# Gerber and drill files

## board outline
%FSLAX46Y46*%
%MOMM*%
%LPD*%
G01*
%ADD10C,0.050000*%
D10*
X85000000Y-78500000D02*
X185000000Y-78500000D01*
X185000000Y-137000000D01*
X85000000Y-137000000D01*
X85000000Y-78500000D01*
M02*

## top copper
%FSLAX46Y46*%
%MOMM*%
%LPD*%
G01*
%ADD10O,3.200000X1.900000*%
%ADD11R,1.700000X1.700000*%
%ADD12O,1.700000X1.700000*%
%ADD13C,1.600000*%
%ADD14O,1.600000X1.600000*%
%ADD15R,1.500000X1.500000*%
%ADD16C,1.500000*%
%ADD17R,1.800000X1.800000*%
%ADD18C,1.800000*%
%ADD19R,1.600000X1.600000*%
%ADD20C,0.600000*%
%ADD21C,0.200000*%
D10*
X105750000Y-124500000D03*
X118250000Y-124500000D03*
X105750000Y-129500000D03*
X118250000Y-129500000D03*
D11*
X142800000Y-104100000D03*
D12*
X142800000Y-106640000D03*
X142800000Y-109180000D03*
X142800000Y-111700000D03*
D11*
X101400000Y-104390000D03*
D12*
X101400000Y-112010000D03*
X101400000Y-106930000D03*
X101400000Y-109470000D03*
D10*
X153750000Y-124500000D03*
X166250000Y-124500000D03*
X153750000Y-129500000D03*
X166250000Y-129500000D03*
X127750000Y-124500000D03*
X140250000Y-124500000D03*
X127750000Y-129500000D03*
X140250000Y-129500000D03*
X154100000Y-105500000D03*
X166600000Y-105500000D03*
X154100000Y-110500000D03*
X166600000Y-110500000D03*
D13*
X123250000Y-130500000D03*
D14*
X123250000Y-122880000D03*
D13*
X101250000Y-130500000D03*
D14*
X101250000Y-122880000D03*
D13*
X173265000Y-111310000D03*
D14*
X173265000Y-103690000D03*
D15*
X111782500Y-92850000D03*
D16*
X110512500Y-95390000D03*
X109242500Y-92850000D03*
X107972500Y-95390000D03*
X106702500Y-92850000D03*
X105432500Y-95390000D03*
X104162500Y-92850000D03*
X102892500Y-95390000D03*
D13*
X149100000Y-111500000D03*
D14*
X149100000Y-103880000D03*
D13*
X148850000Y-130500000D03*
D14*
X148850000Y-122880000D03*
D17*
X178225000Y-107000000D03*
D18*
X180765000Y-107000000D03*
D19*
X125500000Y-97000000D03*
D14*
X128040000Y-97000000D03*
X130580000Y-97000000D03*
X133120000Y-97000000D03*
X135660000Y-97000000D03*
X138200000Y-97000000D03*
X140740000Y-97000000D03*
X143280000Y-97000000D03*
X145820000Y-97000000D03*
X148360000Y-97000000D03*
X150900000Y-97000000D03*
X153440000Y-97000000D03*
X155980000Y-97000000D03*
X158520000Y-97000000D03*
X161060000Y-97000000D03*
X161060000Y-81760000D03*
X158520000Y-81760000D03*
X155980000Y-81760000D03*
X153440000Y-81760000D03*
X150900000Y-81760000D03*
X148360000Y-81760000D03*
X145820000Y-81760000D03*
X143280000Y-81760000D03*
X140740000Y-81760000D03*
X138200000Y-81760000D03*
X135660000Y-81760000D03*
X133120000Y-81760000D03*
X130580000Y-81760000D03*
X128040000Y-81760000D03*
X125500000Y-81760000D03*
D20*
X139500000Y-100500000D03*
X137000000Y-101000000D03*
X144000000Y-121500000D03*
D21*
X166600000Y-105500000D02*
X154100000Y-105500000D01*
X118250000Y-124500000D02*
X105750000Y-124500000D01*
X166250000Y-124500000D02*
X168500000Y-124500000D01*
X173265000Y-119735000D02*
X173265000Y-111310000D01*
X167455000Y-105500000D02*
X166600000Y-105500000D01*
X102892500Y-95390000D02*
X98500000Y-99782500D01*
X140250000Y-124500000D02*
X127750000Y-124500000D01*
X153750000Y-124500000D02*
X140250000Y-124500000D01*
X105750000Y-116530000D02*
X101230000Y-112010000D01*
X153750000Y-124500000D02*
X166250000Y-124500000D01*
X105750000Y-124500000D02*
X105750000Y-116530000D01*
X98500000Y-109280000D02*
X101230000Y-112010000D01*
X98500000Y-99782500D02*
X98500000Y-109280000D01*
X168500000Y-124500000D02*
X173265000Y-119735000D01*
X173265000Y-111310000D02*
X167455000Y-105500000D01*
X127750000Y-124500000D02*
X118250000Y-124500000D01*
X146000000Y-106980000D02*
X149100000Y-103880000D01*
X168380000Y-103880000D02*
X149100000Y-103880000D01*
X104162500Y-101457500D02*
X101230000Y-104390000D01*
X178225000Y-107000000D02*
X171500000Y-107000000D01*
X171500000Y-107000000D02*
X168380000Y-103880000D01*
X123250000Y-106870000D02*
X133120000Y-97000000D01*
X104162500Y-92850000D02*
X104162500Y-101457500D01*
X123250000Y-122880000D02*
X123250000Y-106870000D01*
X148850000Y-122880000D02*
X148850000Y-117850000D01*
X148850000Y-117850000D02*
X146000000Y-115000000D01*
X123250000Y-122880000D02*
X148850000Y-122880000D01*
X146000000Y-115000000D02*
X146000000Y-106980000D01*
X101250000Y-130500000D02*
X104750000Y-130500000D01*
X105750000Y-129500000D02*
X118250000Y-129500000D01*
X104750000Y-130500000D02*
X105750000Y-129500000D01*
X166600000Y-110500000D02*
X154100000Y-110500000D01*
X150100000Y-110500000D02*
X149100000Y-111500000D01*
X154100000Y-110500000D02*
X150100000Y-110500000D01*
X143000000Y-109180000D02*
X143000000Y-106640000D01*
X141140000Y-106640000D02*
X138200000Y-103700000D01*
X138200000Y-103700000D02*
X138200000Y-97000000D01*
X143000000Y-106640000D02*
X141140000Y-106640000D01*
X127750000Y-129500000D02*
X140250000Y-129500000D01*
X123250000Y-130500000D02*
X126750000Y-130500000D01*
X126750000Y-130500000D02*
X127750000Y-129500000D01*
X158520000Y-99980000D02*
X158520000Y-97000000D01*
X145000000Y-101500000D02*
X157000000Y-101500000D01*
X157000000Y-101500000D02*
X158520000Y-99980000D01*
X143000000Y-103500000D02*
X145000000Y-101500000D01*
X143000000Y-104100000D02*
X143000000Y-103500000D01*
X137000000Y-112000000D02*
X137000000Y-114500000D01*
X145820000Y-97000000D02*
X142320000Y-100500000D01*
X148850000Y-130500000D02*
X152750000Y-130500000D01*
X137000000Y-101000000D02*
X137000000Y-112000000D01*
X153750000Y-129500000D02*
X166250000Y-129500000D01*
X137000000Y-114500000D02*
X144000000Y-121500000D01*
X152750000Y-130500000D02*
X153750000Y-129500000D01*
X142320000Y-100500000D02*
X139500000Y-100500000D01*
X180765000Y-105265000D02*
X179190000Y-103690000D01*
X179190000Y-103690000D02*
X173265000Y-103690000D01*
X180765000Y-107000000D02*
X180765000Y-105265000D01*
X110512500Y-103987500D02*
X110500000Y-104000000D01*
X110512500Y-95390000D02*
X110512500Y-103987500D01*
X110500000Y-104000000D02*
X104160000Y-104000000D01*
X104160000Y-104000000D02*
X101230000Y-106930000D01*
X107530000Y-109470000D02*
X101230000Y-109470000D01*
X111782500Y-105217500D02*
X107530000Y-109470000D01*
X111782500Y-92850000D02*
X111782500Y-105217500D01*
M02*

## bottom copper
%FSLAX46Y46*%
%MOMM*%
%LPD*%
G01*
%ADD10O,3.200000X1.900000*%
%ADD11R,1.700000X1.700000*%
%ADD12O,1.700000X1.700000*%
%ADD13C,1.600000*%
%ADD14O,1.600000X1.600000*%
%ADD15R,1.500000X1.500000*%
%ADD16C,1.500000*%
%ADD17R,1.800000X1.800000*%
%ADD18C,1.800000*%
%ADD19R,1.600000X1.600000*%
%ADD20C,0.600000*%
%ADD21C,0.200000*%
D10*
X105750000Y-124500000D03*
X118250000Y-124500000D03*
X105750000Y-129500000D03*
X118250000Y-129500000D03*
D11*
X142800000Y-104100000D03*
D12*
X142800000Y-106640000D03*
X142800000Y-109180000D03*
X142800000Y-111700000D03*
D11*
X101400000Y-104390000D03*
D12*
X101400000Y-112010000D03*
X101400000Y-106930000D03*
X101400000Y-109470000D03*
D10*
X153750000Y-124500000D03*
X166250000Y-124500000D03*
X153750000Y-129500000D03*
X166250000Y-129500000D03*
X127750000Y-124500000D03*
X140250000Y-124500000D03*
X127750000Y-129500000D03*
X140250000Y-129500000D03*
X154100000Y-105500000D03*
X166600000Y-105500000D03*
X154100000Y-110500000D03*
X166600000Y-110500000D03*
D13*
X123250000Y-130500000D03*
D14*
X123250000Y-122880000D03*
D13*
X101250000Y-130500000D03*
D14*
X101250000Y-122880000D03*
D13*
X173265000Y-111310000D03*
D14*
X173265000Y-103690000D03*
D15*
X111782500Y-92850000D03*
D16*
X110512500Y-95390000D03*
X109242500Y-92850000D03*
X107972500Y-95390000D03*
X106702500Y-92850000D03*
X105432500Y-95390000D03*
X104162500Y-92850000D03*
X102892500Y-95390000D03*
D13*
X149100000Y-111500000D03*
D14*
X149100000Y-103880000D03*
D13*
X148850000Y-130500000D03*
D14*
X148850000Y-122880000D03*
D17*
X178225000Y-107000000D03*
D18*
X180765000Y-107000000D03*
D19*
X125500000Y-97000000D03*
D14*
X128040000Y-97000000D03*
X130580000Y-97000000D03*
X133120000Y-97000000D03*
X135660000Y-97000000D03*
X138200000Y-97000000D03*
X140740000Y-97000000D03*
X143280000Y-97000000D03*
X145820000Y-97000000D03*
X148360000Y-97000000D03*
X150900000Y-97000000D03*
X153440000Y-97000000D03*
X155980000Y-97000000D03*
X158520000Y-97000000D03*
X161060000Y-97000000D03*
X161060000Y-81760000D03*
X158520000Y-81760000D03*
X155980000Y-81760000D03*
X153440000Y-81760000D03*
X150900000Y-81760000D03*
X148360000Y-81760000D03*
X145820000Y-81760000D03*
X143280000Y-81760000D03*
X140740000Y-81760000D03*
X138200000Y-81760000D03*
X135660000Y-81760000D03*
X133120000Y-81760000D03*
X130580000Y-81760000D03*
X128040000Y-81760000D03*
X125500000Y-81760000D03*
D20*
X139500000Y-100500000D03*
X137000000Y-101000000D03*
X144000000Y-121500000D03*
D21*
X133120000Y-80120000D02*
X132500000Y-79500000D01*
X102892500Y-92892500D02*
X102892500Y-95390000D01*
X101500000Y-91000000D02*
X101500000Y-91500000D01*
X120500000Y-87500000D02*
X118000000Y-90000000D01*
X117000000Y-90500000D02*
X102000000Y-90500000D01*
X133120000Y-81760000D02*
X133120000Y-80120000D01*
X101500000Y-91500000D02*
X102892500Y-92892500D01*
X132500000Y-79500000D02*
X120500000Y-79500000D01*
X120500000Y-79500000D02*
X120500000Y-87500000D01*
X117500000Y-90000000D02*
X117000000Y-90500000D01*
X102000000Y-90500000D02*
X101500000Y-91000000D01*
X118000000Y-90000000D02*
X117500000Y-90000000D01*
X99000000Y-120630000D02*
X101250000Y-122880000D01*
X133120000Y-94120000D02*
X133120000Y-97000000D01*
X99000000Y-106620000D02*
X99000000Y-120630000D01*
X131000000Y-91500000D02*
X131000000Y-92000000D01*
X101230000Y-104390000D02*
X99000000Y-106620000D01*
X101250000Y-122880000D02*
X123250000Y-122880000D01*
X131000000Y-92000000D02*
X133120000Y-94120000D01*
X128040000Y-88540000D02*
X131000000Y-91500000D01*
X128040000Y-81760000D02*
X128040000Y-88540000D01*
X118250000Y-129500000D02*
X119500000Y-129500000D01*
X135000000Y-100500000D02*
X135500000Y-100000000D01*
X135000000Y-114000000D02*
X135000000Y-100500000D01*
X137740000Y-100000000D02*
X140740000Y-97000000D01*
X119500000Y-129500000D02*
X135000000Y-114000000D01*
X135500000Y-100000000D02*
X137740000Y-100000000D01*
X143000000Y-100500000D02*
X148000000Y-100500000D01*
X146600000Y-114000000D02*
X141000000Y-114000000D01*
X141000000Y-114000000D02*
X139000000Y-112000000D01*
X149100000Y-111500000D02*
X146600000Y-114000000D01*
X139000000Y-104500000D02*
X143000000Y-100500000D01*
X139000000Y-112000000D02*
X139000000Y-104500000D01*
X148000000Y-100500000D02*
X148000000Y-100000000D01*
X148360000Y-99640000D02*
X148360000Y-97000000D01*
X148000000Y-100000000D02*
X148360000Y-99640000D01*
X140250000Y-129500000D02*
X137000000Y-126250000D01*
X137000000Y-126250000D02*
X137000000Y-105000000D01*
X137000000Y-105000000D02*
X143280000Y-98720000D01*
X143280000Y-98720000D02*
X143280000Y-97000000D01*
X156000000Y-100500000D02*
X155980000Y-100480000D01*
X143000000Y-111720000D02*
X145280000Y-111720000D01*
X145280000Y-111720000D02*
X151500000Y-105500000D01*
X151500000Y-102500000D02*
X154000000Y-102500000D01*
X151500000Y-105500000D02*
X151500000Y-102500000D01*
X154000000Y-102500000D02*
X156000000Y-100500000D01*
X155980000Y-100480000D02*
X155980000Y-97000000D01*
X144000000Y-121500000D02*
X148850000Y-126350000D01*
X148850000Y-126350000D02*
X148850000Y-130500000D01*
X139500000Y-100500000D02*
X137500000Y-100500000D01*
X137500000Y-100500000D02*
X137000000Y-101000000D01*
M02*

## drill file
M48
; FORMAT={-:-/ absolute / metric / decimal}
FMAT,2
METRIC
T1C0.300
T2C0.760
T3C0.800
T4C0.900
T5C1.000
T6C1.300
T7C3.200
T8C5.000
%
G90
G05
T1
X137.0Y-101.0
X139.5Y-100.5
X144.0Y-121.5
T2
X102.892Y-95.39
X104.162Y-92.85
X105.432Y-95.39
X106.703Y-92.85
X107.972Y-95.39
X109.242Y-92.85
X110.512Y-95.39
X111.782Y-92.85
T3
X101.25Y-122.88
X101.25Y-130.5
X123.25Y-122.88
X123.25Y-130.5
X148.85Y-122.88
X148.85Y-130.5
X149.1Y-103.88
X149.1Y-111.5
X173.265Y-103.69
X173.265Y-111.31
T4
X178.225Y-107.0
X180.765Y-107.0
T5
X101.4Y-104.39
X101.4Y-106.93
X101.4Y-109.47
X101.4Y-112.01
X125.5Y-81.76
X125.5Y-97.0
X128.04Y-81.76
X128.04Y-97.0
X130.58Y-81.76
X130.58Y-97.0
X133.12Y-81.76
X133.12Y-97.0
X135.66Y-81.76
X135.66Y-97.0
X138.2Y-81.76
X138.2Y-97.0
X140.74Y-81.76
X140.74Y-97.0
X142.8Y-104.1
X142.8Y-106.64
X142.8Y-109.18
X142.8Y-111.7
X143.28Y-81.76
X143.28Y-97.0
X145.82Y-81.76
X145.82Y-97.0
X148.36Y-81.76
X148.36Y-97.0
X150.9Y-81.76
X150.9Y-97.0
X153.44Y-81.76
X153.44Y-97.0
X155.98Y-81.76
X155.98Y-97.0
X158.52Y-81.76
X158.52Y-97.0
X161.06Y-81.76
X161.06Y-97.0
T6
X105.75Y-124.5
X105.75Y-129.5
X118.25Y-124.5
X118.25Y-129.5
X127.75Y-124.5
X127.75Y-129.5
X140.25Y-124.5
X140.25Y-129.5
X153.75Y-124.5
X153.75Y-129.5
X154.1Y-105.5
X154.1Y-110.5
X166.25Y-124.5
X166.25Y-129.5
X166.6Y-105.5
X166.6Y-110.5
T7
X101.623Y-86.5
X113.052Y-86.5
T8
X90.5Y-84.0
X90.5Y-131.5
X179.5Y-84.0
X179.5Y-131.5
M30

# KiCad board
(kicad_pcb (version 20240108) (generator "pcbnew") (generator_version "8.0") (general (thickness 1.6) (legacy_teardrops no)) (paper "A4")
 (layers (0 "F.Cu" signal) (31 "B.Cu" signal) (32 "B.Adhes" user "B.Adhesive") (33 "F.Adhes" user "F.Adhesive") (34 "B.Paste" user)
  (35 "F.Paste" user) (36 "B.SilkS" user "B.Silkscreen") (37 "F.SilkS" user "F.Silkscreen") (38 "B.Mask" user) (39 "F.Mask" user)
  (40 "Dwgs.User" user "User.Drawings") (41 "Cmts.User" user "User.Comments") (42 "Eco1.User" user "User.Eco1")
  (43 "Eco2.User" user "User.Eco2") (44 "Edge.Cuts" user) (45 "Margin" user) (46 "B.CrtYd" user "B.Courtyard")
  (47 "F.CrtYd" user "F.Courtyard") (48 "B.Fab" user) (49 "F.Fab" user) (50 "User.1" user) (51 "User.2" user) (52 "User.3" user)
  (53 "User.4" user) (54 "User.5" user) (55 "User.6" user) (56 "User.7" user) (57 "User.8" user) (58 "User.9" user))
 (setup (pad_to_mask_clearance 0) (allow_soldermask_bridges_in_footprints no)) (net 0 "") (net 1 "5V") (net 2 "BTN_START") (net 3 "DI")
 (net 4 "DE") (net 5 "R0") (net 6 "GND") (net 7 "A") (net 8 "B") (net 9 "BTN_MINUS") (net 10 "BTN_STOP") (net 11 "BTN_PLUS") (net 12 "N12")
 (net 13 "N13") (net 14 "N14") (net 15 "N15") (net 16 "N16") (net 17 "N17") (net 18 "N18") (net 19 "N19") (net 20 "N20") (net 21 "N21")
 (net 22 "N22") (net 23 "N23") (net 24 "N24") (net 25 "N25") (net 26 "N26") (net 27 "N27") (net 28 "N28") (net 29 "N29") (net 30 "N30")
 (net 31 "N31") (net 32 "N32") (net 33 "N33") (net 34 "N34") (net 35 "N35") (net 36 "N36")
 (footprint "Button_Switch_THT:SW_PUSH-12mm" (layer "F.Cu") (at 105.75 124.5)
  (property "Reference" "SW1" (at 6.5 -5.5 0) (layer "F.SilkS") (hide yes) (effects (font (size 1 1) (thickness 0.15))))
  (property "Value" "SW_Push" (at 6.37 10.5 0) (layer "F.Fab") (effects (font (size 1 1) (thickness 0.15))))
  (pad "1" thru_hole oval (at 0 0) (size 3.2 1.9) (drill 1.3) (layers "*.Cu" "*.Mask") (remove_unused_layers no) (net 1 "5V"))
  (pad "1" thru_hole oval (at 12.5 0) (size 3.2 1.9) (drill 1.3) (layers "*.Cu" "*.Mask") (remove_unused_layers no) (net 1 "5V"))
  (pad "2" thru_hole oval (at 0 5) (size 3.2 1.9) (drill 1.3) (layers "*.Cu" "*.Mask") (remove_unused_layers no) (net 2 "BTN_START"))
  (pad "2" thru_hole oval (at 12.5 5) (size 3.2 1.9) (drill 1.3) (layers "*.Cu" "*.Mask") (remove_unused_layers no) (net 2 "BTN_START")))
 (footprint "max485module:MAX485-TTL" (layer "F.Cu") (at 117.5 113.5)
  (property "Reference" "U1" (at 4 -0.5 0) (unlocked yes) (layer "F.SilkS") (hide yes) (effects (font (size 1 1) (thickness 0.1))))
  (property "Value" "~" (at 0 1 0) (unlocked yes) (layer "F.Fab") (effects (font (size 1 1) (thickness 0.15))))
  (pad "1" thru_hole rect (at 25.3 -9.4) (size 1.7 1.7) (drill 1) (layers "*.Cu" "*.Mask") (remove_unused_layers no) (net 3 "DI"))
  (pad "2" thru_hole oval (at 25.3 -6.86) (size 1.7 1.7) (drill 1) (layers "*.Cu" "*.Mask") (remove_unused_layers no) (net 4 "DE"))
  (pad "3" thru_hole oval (at 25.3 -4.32) (size 1.7 1.7) (drill 1) (layers "*.Cu" "*.Mask") (remove_unused_layers no) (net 4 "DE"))
  (pad "4" thru_hole oval (at 25.3 -1.8) (size 1.7 1.7) (drill 1) (layers "*.Cu" "*.Mask") (remove_unused_layers no) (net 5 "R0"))
  (pad "5" thru_hole rect (at -16.1 -9.11) (size 1.7 1.7) (drill 1) (layers "*.Cu" "*.Mask") (remove_unused_layers no) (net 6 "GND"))
  (pad "6" thru_hole oval (at -16.1 -1.49) (size 1.7 1.7) (drill 1) (layers "*.Cu" "*.Mask") (remove_unused_layers no) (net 1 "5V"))
  (pad "7" thru_hole oval (at -16.1 -6.57) (size 1.7 1.7) (drill 1) (layers "*.Cu" "*.Mask") (remove_unused_layers no) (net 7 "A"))
  (pad "8" thru_hole oval (at -16.1 -4.03) (size 1.7 1.7) (drill 1) (layers "*.Cu" "*.Mask") (remove_unused_layers no) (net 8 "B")))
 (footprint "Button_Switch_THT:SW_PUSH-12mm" (layer "F.Cu") (at 153.75 124.5)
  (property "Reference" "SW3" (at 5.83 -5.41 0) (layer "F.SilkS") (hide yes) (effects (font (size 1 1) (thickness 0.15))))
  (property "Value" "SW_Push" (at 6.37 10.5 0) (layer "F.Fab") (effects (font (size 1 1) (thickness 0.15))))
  (pad "1" thru_hole oval (at 0 0) (size 3.2 1.9) (drill 1.3) (layers "*.Cu" "*.Mask") (remove_unused_layers no) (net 1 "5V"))
  (pad "1" thru_hole oval (at 12.5 0) (size 3.2 1.9) (drill 1.3) (layers "*.Cu" "*.Mask") (remove_unused_layers no) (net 1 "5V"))
  (pad "2" thru_hole oval (at 0 5) (size 3.2 1.9) (drill 1.3) (layers "*.Cu" "*.Mask") (remove_unused_layers no) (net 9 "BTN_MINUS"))
  (pad "2" thru_hole oval (at 12.5 5) (size 3.2 1.9) (drill 1.3) (layers "*.Cu" "*.Mask") (remove_unused_layers no) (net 9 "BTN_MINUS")))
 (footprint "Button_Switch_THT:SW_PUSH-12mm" (layer "F.Cu") (at 127.75 124.5)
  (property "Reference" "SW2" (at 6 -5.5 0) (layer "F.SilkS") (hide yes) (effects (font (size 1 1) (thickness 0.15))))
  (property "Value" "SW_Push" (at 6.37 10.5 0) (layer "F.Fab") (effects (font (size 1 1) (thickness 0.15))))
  (pad "1" thru_hole oval (at 0 0) (size 3.2 1.9) (drill 1.3) (layers "*.Cu" "*.Mask") (remove_unused_layers no) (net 1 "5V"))
  (pad "1" thru_hole oval (at 12.5 0) (size 3.2 1.9) (drill 1.3) (layers "*.Cu" "*.Mask") (remove_unused_layers no) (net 1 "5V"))
  (pad "2" thru_hole oval (at 0 5) (size 3.2 1.9) (drill 1.3) (layers "*.Cu" "*.Mask") (remove_unused_layers no) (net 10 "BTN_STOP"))
  (pad "2" thru_hole oval (at 12.5 5) (size 3.2 1.9) (drill 1.3) (layers "*.Cu" "*.Mask") (remove_unused_layers no) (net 10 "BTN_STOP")))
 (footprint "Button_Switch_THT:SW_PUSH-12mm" (layer "F.Cu") (at 154.1 105.5)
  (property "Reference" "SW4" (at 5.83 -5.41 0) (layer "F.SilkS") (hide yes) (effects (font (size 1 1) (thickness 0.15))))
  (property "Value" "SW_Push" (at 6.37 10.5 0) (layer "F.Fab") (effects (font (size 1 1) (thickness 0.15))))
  (pad "1" thru_hole oval (at 0 0) (size 3.2 1.9) (drill 1.3) (layers "*.Cu" "*.Mask") (remove_unused_layers no) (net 1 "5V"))
  (pad "1" thru_hole oval (at 12.5 0) (size 3.2 1.9) (drill 1.3) (layers "*.Cu" "*.Mask") (remove_unused_layers no) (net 1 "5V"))
  (pad "2" thru_hole oval (at 0 5) (size 3.2 1.9) (drill 1.3) (layers "*.Cu" "*.Mask") (remove_unused_layers no) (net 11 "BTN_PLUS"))
  (pad "2" thru_hole oval (at 12.5 5) (size 3.2 1.9) (drill 1.3) (layers "*.Cu" "*.Mask") (remove_unused_layers no) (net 11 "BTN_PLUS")))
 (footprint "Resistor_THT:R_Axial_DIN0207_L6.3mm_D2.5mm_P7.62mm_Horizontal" (layer "F.Cu") (at 123.25 130.5 90)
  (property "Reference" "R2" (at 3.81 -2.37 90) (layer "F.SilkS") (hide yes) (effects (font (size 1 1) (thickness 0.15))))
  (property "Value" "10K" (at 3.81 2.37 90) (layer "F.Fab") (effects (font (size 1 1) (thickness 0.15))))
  (pad "1" thru_hole circle (at 0 0 90) (size 1.6 1.6) (drill 0.8) (layers "*.Cu" "*.Mask") (remove_unused_layers no) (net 10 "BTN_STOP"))
  (pad "2" thru_hole oval (at 7.62 0 90) (size 1.6 1.6) (drill 0.8) (layers "*.Cu" "*.Mask") (remove_unused_layers no) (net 6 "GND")))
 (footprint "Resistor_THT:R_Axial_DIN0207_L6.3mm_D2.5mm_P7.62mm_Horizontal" (layer "F.Cu") (at 101.25 130.5 90)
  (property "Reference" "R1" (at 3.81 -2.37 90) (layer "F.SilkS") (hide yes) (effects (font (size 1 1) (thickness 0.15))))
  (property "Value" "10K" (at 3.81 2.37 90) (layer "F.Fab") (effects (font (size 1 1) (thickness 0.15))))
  (pad "1" thru_hole circle (at 0 0 90) (size 1.6 1.6) (drill 0.8) (layers "*.Cu" "*.Mask") (remove_unused_layers no) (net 2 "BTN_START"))
  (pad "2" thru_hole oval (at 7.62 0 90) (size 1.6 1.6) (drill 0.8) (layers "*.Cu" "*.Mask") (remove_unused_layers no) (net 6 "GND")))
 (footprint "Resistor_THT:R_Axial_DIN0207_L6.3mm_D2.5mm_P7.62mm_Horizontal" (layer "F.Cu") (at 173.265 111.31 90)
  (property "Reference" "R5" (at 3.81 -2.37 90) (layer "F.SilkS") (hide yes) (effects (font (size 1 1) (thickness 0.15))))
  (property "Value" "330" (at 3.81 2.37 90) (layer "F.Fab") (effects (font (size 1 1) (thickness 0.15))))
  (pad "1" thru_hole circle (at 0 0 90) (size 1.6 1.6) (drill 0.8) (layers "*.Cu" "*.Mask") (remove_unused_layers no) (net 1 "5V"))
  (pad "2" thru_hole oval (at 7.62 0 90) (size 1.6 1.6) (drill 0.8) (layers "*.Cu" "*.Mask") (remove_unused_layers no) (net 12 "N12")))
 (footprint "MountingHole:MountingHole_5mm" (layer "F.Cu") (at 90.5 131.5)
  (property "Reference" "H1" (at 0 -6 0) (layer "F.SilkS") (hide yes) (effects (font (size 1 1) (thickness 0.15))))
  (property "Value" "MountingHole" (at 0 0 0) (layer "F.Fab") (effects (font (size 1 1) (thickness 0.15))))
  (pad "" np_thru_hole circle (at 0 0) (size 5 5) (drill 5) (layers "*.Cu" "*.Mask")))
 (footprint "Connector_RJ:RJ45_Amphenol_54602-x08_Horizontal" (layer "F.Cu") (at 111.7825 92.85 180)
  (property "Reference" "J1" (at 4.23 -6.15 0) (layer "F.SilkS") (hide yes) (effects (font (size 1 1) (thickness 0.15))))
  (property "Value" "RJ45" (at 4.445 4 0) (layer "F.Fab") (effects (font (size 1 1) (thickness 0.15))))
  (pad "" np_thru_hole circle (at -1.27 6.35 180) (size 3.2 3.2) (drill 3.2) (layers "*.Cu" "*.Mask"))
  (pad "" np_thru_hole circle (at 10.16 6.35 180) (size 3.2 3.2) (drill 3.2) (layers "*.Cu" "*.Mask"))
  (pad "1" thru_hole rect (at 0 0 180) (size 1.5 1.5) (drill 0.76) (layers "*.Cu" "*.Mask") (remove_unused_layers no) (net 8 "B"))
  (pad "2" thru_hole circle (at 1.27 -2.54 180) (size 1.5 1.5) (drill 0.76) (layers "*.Cu" "*.Mask") (remove_unused_layers no) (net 7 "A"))
  (pad "3" thru_hole circle (at 2.54 0 180) (size 1.5 1.5) (drill 0.76) (layers "*.Cu" "*.Mask") (remove_unused_layers no) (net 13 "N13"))
  (pad "4" thru_hole circle (at 3.81 -2.54 180) (size 1.5 1.5) (drill 0.76) (layers "*.Cu" "*.Mask") (remove_unused_layers no)
   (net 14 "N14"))
  (pad "5" thru_hole circle (at 5.08 0 180) (size 1.5 1.5) (drill 0.76) (layers "*.Cu" "*.Mask") (remove_unused_layers no) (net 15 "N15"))
  (pad "6" thru_hole circle (at 6.35 -2.54 180) (size 1.5 1.5) (drill 0.76) (layers "*.Cu" "*.Mask") (remove_unused_layers no)
   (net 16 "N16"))
  (pad "7" thru_hole circle (at 7.62 0 180) (size 1.5 1.5) (drill 0.76) (layers "*.Cu" "*.Mask") (remove_unused_layers no) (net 6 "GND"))
  (pad "8" thru_hole circle (at 8.89 -2.54 180) (size 1.5 1.5) (drill 0.76) (layers "*.Cu" "*.Mask") (remove_unused_layers no) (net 1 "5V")))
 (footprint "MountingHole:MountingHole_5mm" (layer "F.Cu") (at 90.5 84)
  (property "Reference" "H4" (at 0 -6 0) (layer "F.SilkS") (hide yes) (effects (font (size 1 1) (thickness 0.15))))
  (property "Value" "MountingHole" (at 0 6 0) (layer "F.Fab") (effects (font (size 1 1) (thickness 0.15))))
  (pad "" np_thru_hole circle (at 0 0) (size 5 5) (drill 5) (layers "*.Cu" "*.Mask")))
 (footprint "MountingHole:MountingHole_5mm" (layer "F.Cu") (at 179.5 131.5)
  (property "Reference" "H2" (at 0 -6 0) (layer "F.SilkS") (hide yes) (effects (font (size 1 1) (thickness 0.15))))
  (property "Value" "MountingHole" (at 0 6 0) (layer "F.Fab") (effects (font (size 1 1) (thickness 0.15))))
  (pad "" np_thru_hole circle (at 0 0) (size 5 5) (drill 5) (layers "*.Cu" "*.Mask")))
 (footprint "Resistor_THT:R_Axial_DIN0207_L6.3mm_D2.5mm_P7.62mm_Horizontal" (layer "F.Cu") (at 149.1 111.5 90)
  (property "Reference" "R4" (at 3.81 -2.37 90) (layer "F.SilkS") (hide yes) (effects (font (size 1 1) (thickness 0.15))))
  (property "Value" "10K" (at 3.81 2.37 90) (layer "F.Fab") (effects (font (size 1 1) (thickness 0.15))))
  (pad "1" thru_hole circle (at 0 0 90) (size 1.6 1.6) (drill 0.8) (layers "*.Cu" "*.Mask") (remove_unused_layers no) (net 11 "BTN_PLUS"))
  (pad "2" thru_hole oval (at 7.62 0 90) (size 1.6 1.6) (drill 0.8) (layers "*.Cu" "*.Mask") (remove_unused_layers no) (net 6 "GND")))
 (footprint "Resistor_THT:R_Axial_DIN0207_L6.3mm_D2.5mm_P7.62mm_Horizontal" (layer "F.Cu") (at 148.85 130.5 90)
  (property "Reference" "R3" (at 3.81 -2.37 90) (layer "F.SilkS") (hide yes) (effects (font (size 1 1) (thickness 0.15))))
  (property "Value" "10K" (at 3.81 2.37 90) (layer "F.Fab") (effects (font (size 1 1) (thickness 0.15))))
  (pad "1" thru_hole circle (at 0 0 90) (size 1.6 1.6) (drill 0.8) (layers "*.Cu" "*.Mask") (remove_unused_layers no) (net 9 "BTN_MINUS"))
  (pad "2" thru_hole oval (at 7.62 0 90) (size 1.6 1.6) (drill 0.8) (layers "*.Cu" "*.Mask") (remove_unused_layers no) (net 6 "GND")))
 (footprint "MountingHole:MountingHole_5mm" (layer "F.Cu") (at 179.5 84)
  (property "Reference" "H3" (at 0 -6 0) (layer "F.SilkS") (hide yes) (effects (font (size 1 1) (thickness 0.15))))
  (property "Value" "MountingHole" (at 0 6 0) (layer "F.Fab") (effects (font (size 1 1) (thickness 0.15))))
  (pad "" np_thru_hole circle (at 0 0) (size 5 5) (drill 5) (layers "*.Cu" "*.Mask")))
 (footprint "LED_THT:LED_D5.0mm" (layer "F.Cu") (at 178.225 107)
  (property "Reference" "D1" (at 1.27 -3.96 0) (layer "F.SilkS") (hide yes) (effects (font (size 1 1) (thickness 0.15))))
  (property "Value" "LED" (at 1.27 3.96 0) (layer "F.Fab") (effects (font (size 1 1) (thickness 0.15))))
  (pad "1" thru_hole rect (at 0 0) (size 1.8 1.8) (drill 0.9) (layers "*.Cu" "*.Mask") (remove_unused_layers no) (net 6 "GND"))
  (pad "2" thru_hole circle (at 2.54 0) (size 1.8 1.8) (drill 0.9) (layers "*.Cu" "*.Mask") (remove_unused_layers no) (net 12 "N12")))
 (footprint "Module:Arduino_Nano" (layer "F.Cu") (at 125.5 97 90)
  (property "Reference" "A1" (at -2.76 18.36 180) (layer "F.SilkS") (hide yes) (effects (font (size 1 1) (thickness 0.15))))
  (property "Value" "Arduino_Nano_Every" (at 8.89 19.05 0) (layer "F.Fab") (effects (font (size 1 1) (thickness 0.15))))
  (pad "1" thru_hole rect (at 0 0 90) (size 1.6 1.6) (drill 1) (layers "*.Cu" "*.Mask") (remove_unused_layers no) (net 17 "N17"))
  (pad "2" thru_hole oval (at 0 2.54 90) (size 1.6 1.6) (drill 1) (layers "*.Cu" "*.Mask") (remove_unused_layers no) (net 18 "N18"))
  (pad "3" thru_hole oval (at 0 5.08 90) (size 1.6 1.6) (drill 1) (layers "*.Cu" "*.Mask") (remove_unused_layers no) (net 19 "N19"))
  (pad "4" thru_hole oval (at 0 7.62 90) (size 1.6 1.6) (drill 1) (layers "*.Cu" "*.Mask") (remove_unused_layers no) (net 6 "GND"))
  (pad "5" thru_hole oval (at 0 10.16 90) (size 1.6 1.6) (drill 1) (layers "*.Cu" "*.Mask") (remove_unused_layers no) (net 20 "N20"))
  (pad "6" thru_hole oval (at 0 12.7 90) (size 1.6 1.6) (drill 1) (layers "*.Cu" "*.Mask") (remove_unused_layers no) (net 4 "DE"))
  (pad "7" thru_hole oval (at 0 15.24 90) (size 1.6 1.6) (drill 1) (layers "*.Cu" "*.Mask") (remove_unused_layers no) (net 2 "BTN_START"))
  (pad "8" thru_hole oval (at 0 17.78 90) (size 1.6 1.6) (drill 1) (layers "*.Cu" "*.Mask") (remove_unused_layers no) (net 10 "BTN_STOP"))
  (pad "9" thru_hole oval (at 0 20.32 90) (size 1.6 1.6) (drill 1) (layers "*.Cu" "*.Mask") (remove_unused_layers no) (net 9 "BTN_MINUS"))
  (pad "10" thru_hole oval (at 0 22.86 90) (size 1.6 1.6) (drill 1) (layers "*.Cu" "*.Mask") (remove_unused_layers no) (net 11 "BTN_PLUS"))
  (pad "11" thru_hole oval (at 0 25.4 90) (size 1.6 1.6) (drill 1) (layers "*.Cu" "*.Mask") (remove_unused_layers no) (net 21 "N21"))
  (pad "12" thru_hole oval (at 0 27.94 90) (size 1.6 1.6) (drill 1) (layers "*.Cu" "*.Mask") (remove_unused_layers no) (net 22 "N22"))
  (pad "13" thru_hole oval (at 0 30.48 90) (size 1.6 1.6) (drill 1) (layers "*.Cu" "*.Mask") (remove_unused_layers no) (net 5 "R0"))
  (pad "14" thru_hole oval (at 0 33.02 90) (size 1.6 1.6) (drill 1) (layers "*.Cu" "*.Mask") (remove_unused_layers no) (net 3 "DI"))
  (pad "15" thru_hole oval (at 0 35.56 90) (size 1.6 1.6) (drill 1) (layers "*.Cu" "*.Mask") (remove_unused_layers no) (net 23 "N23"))
  (pad "16" thru_hole oval (at 15.24 35.56 90) (size 1.6 1.6) (drill 1) (layers "*.Cu" "*.Mask") (remove_unused_layers no) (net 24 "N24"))
  (pad "17" thru_hole oval (at 15.24 33.02 90) (size 1.6 1.6) (drill 1) (layers "*.Cu" "*.Mask") (remove_unused_layers no) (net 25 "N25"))
  (pad "18" thru_hole oval (at 15.24 30.48 90) (size 1.6 1.6) (drill 1) (layers "*.Cu" "*.Mask") (remove_unused_layers no) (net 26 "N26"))
  (pad "19" thru_hole oval (at 15.24 27.94 90) (size 1.6 1.6) (drill 1) (layers "*.Cu" "*.Mask") (remove_unused_layers no) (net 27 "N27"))
  (pad "20" thru_hole oval (at 15.24 25.4 90) (size 1.6 1.6) (drill 1) (layers "*.Cu" "*.Mask") (remove_unused_layers no) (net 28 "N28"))
  (pad "21" thru_hole oval (at 15.24 22.86 90) (size 1.6 1.6) (drill 1) (layers "*.Cu" "*.Mask") (remove_unused_layers no) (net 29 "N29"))
  (pad "22" thru_hole oval (at 15.24 20.32 90) (size 1.6 1.6) (drill 1) (layers "*.Cu" "*.Mask") (remove_unused_layers no) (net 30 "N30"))
  (pad "23" thru_hole oval (at 15.24 17.78 90) (size 1.6 1.6) (drill 1) (layers "*.Cu" "*.Mask") (remove_unused_layers no) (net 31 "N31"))
  (pad "24" thru_hole oval (at 15.24 15.24 90) (size 1.6 1.6) (drill 1) (layers "*.Cu" "*.Mask") (remove_unused_layers no) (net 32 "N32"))
  (pad "25" thru_hole oval (at 15.24 12.7 90) (size 1.6 1.6) (drill 1) (layers "*.Cu" "*.Mask") (remove_unused_layers no) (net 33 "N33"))
  (pad "26" thru_hole oval (at 15.24 10.16 90) (size 1.6 1.6) (drill 1) (layers "*.Cu" "*.Mask") (remove_unused_layers no) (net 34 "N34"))
  (pad "27" thru_hole oval (at 15.24 7.62 90) (size 1.6 1.6) (drill 1) (layers "*.Cu" "*.Mask") (remove_unused_layers no) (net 1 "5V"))
  (pad "28" thru_hole oval (at 15.24 5.08 90) (size 1.6 1.6) (drill 1) (layers "*.Cu" "*.Mask") (remove_unused_layers no) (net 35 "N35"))
  (pad "29" thru_hole oval (at 15.24 2.54 90) (size 1.6 1.6) (drill 1) (layers "*.Cu" "*.Mask") (remove_unused_layers no) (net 6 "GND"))
  (pad "30" thru_hole oval (at 15.24 0 90) (size 1.6 1.6) (drill 1) (layers "*.Cu" "*.Mask") (remove_unused_layers no) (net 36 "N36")))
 (gr_rect (start 85 78.5) (end 185 137) (stroke (width 0.05) (type default)) (fill none) (layer "Edge.Cuts"))
 (segment (start 166.6 105.5) (end 154.1 105.5) (width 0.2) (layer "F.Cu") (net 1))
 (segment (start 118.25 124.5) (end 105.75 124.5) (width 0.2) (layer "F.Cu") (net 1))
 (segment (start 166.25 124.5) (end 168.5 124.5) (width 0.2) (layer "F.Cu") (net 1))
 (segment (start 173.265 119.735) (end 173.265 111.31) (width 0.2) (layer "F.Cu") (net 1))
 (segment (start 167.455 105.5) (end 166.6 105.5) (width 0.2) (layer "F.Cu") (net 1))
 (segment (start 102.8925 95.39) (end 98.5 99.7825) (width 0.2) (layer "F.Cu") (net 1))
 (segment (start 140.25 124.5) (end 127.75 124.5) (width 0.2) (layer "F.Cu") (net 1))
 (segment (start 153.75 124.5) (end 140.25 124.5) (width 0.2) (layer "F.Cu") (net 1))
 (segment (start 105.75 116.53) (end 101.23 112.01) (width 0.2) (layer "F.Cu") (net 1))
 (segment (start 153.75 124.5) (end 166.25 124.5) (width 0.2) (layer "F.Cu") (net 1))
 (segment (start 105.75 124.5) (end 105.75 116.53) (width 0.2) (layer "F.Cu") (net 1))
 (segment (start 98.5 109.28) (end 101.23 112.01) (width 0.2) (layer "F.Cu") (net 1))
 (segment (start 98.5 99.7825) (end 98.5 109.28) (width 0.2) (layer "F.Cu") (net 1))
 (segment (start 168.5 124.5) (end 173.265 119.735) (width 0.2) (layer "F.Cu") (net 1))
 (segment (start 173.265 111.31) (end 167.455 105.5) (width 0.2) (layer "F.Cu") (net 1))
 (segment (start 127.75 124.5) (end 118.25 124.5) (width 0.2) (layer "F.Cu") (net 1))
 (segment (start 133.12 80.12) (end 132.5 79.5) (width 0.2) (layer "B.Cu") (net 1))
 (segment (start 102.8925 92.8925) (end 102.8925 95.39) (width 0.2) (layer "B.Cu") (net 1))
 (segment (start 101.5 91) (end 101.5 91.5) (width 0.2) (layer "B.Cu") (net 1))
 (segment (start 120.5 87.5) (end 118 90) (width 0.2) (layer "B.Cu") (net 1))
 (segment (start 117 90.5) (end 102 90.5) (width 0.2) (layer "B.Cu") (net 1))
 (segment (start 133.12 81.76) (end 133.12 80.12) (width 0.2) (layer "B.Cu") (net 1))
 (segment (start 101.5 91.5) (end 102.8925 92.8925) (width 0.2) (layer "B.Cu") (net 1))
 (segment (start 132.5 79.5) (end 120.5 79.5) (width 0.2) (layer "B.Cu") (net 1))
 (segment (start 120.5 79.5) (end 120.5 87.5) (width 0.2) (layer "B.Cu") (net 1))
 (segment (start 117.5 90) (end 117 90.5) (width 0.2) (layer "B.Cu") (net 1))
 (segment (start 102 90.5) (end 101.5 91) (width 0.2) (layer "B.Cu") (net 1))
 (segment (start 118 90) (end 117.5 90) (width 0.2) (layer "B.Cu") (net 1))
 (segment (start 146 106.98) (end 149.1 103.88) (width 0.2) (layer "F.Cu") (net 6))
 (segment (start 168.38 103.88) (end 149.1 103.88) (width 0.2) (layer "F.Cu") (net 6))
 (segment (start 104.1625 101.4575) (end 101.23 104.39) (width 0.2) (layer "F.Cu") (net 6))
 (segment (start 178.225 107) (end 171.5 107) (width 0.2) (layer "F.Cu") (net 6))
 (segment (start 171.5 107) (end 168.38 103.88) (width 0.2) (layer "F.Cu") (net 6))
 (segment (start 123.25 106.87) (end 133.12 97) (width 0.2) (layer "F.Cu") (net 6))
 (segment (start 104.1625 92.85) (end 104.1625 101.4575) (width 0.2) (layer "F.Cu") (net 6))
 (segment (start 123.25 122.88) (end 123.25 106.87) (width 0.2) (layer "F.Cu") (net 6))
 (segment (start 148.85 122.88) (end 148.85 117.85) (width 0.2) (layer "F.Cu") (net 6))
 (segment (start 148.85 117.85) (end 146 115) (width 0.2) (layer "F.Cu") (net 6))
 (segment (start 123.25 122.88) (end 148.85 122.88) (width 0.2) (layer "F.Cu") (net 6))
 (segment (start 146 115) (end 146 106.98) (width 0.2) (layer "F.Cu") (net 6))
 (segment (start 99 120.63) (end 101.25 122.88) (width 0.2) (layer "B.Cu") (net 6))
 (segment (start 133.12 94.12) (end 133.12 97) (width 0.2) (layer "B.Cu") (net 6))
 (segment (start 99 106.62) (end 99 120.63) (width 0.2) (layer "B.Cu") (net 6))
 (segment (start 131 91.5) (end 131 92) (width 0.2) (layer "B.Cu") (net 6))
 (segment (start 101.23 104.39) (end 99 106.62) (width 0.2) (layer "B.Cu") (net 6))
 (segment (start 101.25 122.88) (end 123.25 122.88) (width 0.2) (layer "B.Cu") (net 6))
 (segment (start 131 92) (end 133.12 94.12) (width 0.2) (layer "B.Cu") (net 6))
 (segment (start 128.04 88.54) (end 131 91.5) (width 0.2) (layer "B.Cu") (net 6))
 (segment (start 128.04 81.76) (end 128.04 88.54) (width 0.2) (layer "B.Cu") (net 6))
 (segment (start 101.25 130.5) (end 104.75 130.5) (width 0.2) (layer "F.Cu") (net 2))
 (segment (start 105.75 129.5) (end 118.25 129.5) (width 0.2) (layer "F.Cu") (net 2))
 (segment (start 104.75 130.5) (end 105.75 129.5) (width 0.2) (layer "F.Cu") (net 2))
 (segment (start 118.25 129.5) (end 119.5 129.5) (width 0.2) (layer "B.Cu") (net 2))
 (segment (start 135 100.5) (end 135.5 100) (width 0.2) (layer "B.Cu") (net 2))
 (segment (start 135 114) (end 135 100.5) (width 0.2) (layer "B.Cu") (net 2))
 (segment (start 137.74 100) (end 140.74 97) (width 0.2) (layer "B.Cu") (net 2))
 (segment (start 119.5 129.5) (end 135 114) (width 0.2) (layer "B.Cu") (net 2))
 (segment (start 135.5 100) (end 137.74 100) (width 0.2) (layer "B.Cu") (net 2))
 (segment (start 166.6 110.5) (end 154.1 110.5) (width 0.2) (layer "F.Cu") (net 11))
 (segment (start 150.1 110.5) (end 149.1 111.5) (width 0.2) (layer "F.Cu") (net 11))
 (segment (start 154.1 110.5) (end 150.1 110.5) (width 0.2) (layer "F.Cu") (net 11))
 (segment (start 143 100.5) (end 148 100.5) (width 0.2) (layer "B.Cu") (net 11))
 (segment (start 146.6 114) (end 141 114) (width 0.2) (layer "B.Cu") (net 11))
 (segment (start 141 114) (end 139 112) (width 0.2) (layer "B.Cu") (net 11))
 (segment (start 149.1 111.5) (end 146.6 114) (width 0.2) (layer "B.Cu") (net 11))
 (segment (start 139 104.5) (end 143 100.5) (width 0.2) (layer "B.Cu") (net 11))
 (segment (start 139 112) (end 139 104.5) (width 0.2) (layer "B.Cu") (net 11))
 (segment (start 148 100.5) (end 148 100) (width 0.2) (layer "B.Cu") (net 11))
 (segment (start 148.36 99.64) (end 148.36 97) (width 0.2) (layer "B.Cu") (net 11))
 (segment (start 148 100) (end 148.36 99.64) (width 0.2) (layer "B.Cu") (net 11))
 (segment (start 143 109.18) (end 143 106.64) (width 0.2) (layer "F.Cu") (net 4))
 (segment (start 141.14 106.64) (end 138.2 103.7) (width 0.2) (layer "F.Cu") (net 4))
 (segment (start 138.2 103.7) (end 138.2 97) (width 0.2) (layer "F.Cu") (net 4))
 (segment (start 143 106.64) (end 141.14 106.64) (width 0.2) (layer "F.Cu") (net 4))
 (segment (start 127.75 129.5) (end 140.25 129.5) (width 0.2) (layer "F.Cu") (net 10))
 (segment (start 123.25 130.5) (end 126.75 130.5) (width 0.2) (layer "F.Cu") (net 10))
 (segment (start 126.75 130.5) (end 127.75 129.5) (width 0.2) (layer "F.Cu") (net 10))
 (segment (start 140.25 129.5) (end 137 126.25) (width 0.2) (layer "B.Cu") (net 10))
 (segment (start 137 126.25) (end 137 105) (width 0.2) (layer "B.Cu") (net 10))
 (segment (start 137 105) (end 143.28 98.72) (width 0.2) (layer "B.Cu") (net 10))
 (segment (start 143.28 98.72) (end 143.28 97) (width 0.2) (layer "B.Cu") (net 10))
 (segment (start 158.52 99.98) (end 158.52 97) (width 0.2) (layer "F.Cu") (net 3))
 (segment (start 145 101.5) (end 157 101.5) (width 0.2) (layer "F.Cu") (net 3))
 (segment (start 157 101.5) (end 158.52 99.98) (width 0.2) (layer "F.Cu") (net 3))
 (segment (start 143 103.5) (end 145 101.5) (width 0.2) (layer "F.Cu") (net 3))
 (segment (start 143 104.1) (end 143 103.5) (width 0.2) (layer "F.Cu") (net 3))
 (segment (start 156 100.5) (end 155.98 100.48) (width 0.2) (layer "B.Cu") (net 5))
 (segment (start 143 111.72) (end 145.28 111.72) (width 0.2) (layer "B.Cu") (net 5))
 (segment (start 145.28 111.72) (end 151.5 105.5) (width 0.2) (layer "B.Cu") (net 5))
 (segment (start 151.5 102.5) (end 154 102.5) (width 0.2) (layer "B.Cu") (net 5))
 (segment (start 151.5 105.5) (end 151.5 102.5) (width 0.2) (layer "B.Cu") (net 5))
 (segment (start 154 102.5) (end 156 100.5) (width 0.2) (layer "B.Cu") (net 5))
 (segment (start 155.98 100.48) (end 155.98 97) (width 0.2) (layer "B.Cu") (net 5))
 (segment (start 137 112) (end 137 114.5) (width 0.2) (layer "F.Cu") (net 9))
 (segment (start 145.82 97) (end 142.32 100.5) (width 0.2) (layer "F.Cu") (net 9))
 (segment (start 148.85 130.5) (end 152.75 130.5) (width 0.2) (layer "F.Cu") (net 9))
 (segment (start 137 101) (end 137 112) (width 0.2) (layer "F.Cu") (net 9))
 (segment (start 153.75 129.5) (end 166.25 129.5) (width 0.2) (layer "F.Cu") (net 9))
 (segment (start 137 114.5) (end 144 121.5) (width 0.2) (layer "F.Cu") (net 9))
 (segment (start 152.75 130.5) (end 153.75 129.5) (width 0.2) (layer "F.Cu") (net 9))
 (segment (start 142.32 100.5) (end 139.5 100.5) (width 0.2) (layer "F.Cu") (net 9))
 (via (at 139.5 100.5) (size 0.6) (drill 0.3) (layers "F.Cu" "B.Cu") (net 9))
 (via (at 137 101) (size 0.6) (drill 0.3) (layers "F.Cu" "B.Cu") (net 9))
 (via (at 144 121.5) (size 0.6) (drill 0.3) (layers "F.Cu" "B.Cu") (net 9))
 (segment (start 144 121.5) (end 148.85 126.35) (width 0.2) (layer "B.Cu") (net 9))
 (segment (start 148.85 126.35) (end 148.85 130.5) (width 0.2) (layer "B.Cu") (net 9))
 (segment (start 139.5 100.5) (end 137.5 100.5) (width 0.2) (layer "B.Cu") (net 9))
 (segment (start 137.5 100.5) (end 137 101) (width 0.2) (layer "B.Cu") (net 9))
 (segment (start 180.765 105.265) (end 179.19 103.69) (width 0.2) (layer "F.Cu") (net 12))
 (segment (start 179.19 103.69) (end 173.265 103.69) (width 0.2) (layer "F.Cu") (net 12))
 (segment (start 180.765 107) (end 180.765 105.265) (width 0.2) (layer "F.Cu") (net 12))
 (segment (start 110.5125 103.9875) (end 110.5 104) (width 0.2) (layer "F.Cu") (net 7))
 (segment (start 110.5125 95.39) (end 110.5125 103.9875) (width 0.2) (layer "F.Cu") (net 7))
 (segment (start 110.5 104) (end 104.16 104) (width 0.2) (layer "F.Cu") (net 7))
 (segment (start 104.16 104) (end 101.23 106.93) (width 0.2) (layer "F.Cu") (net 7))
 (segment (start 107.53 109.47) (end 101.23 109.47) (width 0.2) (layer "F.Cu") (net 8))
 (segment (start 111.7825 105.2175) (end 107.53 109.47) (width 0.2) (layer "F.Cu") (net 8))
 (segment (start 111.7825 92.85) (end 111.7825 105.2175) (width 0.2) (layer "F.Cu") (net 8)))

